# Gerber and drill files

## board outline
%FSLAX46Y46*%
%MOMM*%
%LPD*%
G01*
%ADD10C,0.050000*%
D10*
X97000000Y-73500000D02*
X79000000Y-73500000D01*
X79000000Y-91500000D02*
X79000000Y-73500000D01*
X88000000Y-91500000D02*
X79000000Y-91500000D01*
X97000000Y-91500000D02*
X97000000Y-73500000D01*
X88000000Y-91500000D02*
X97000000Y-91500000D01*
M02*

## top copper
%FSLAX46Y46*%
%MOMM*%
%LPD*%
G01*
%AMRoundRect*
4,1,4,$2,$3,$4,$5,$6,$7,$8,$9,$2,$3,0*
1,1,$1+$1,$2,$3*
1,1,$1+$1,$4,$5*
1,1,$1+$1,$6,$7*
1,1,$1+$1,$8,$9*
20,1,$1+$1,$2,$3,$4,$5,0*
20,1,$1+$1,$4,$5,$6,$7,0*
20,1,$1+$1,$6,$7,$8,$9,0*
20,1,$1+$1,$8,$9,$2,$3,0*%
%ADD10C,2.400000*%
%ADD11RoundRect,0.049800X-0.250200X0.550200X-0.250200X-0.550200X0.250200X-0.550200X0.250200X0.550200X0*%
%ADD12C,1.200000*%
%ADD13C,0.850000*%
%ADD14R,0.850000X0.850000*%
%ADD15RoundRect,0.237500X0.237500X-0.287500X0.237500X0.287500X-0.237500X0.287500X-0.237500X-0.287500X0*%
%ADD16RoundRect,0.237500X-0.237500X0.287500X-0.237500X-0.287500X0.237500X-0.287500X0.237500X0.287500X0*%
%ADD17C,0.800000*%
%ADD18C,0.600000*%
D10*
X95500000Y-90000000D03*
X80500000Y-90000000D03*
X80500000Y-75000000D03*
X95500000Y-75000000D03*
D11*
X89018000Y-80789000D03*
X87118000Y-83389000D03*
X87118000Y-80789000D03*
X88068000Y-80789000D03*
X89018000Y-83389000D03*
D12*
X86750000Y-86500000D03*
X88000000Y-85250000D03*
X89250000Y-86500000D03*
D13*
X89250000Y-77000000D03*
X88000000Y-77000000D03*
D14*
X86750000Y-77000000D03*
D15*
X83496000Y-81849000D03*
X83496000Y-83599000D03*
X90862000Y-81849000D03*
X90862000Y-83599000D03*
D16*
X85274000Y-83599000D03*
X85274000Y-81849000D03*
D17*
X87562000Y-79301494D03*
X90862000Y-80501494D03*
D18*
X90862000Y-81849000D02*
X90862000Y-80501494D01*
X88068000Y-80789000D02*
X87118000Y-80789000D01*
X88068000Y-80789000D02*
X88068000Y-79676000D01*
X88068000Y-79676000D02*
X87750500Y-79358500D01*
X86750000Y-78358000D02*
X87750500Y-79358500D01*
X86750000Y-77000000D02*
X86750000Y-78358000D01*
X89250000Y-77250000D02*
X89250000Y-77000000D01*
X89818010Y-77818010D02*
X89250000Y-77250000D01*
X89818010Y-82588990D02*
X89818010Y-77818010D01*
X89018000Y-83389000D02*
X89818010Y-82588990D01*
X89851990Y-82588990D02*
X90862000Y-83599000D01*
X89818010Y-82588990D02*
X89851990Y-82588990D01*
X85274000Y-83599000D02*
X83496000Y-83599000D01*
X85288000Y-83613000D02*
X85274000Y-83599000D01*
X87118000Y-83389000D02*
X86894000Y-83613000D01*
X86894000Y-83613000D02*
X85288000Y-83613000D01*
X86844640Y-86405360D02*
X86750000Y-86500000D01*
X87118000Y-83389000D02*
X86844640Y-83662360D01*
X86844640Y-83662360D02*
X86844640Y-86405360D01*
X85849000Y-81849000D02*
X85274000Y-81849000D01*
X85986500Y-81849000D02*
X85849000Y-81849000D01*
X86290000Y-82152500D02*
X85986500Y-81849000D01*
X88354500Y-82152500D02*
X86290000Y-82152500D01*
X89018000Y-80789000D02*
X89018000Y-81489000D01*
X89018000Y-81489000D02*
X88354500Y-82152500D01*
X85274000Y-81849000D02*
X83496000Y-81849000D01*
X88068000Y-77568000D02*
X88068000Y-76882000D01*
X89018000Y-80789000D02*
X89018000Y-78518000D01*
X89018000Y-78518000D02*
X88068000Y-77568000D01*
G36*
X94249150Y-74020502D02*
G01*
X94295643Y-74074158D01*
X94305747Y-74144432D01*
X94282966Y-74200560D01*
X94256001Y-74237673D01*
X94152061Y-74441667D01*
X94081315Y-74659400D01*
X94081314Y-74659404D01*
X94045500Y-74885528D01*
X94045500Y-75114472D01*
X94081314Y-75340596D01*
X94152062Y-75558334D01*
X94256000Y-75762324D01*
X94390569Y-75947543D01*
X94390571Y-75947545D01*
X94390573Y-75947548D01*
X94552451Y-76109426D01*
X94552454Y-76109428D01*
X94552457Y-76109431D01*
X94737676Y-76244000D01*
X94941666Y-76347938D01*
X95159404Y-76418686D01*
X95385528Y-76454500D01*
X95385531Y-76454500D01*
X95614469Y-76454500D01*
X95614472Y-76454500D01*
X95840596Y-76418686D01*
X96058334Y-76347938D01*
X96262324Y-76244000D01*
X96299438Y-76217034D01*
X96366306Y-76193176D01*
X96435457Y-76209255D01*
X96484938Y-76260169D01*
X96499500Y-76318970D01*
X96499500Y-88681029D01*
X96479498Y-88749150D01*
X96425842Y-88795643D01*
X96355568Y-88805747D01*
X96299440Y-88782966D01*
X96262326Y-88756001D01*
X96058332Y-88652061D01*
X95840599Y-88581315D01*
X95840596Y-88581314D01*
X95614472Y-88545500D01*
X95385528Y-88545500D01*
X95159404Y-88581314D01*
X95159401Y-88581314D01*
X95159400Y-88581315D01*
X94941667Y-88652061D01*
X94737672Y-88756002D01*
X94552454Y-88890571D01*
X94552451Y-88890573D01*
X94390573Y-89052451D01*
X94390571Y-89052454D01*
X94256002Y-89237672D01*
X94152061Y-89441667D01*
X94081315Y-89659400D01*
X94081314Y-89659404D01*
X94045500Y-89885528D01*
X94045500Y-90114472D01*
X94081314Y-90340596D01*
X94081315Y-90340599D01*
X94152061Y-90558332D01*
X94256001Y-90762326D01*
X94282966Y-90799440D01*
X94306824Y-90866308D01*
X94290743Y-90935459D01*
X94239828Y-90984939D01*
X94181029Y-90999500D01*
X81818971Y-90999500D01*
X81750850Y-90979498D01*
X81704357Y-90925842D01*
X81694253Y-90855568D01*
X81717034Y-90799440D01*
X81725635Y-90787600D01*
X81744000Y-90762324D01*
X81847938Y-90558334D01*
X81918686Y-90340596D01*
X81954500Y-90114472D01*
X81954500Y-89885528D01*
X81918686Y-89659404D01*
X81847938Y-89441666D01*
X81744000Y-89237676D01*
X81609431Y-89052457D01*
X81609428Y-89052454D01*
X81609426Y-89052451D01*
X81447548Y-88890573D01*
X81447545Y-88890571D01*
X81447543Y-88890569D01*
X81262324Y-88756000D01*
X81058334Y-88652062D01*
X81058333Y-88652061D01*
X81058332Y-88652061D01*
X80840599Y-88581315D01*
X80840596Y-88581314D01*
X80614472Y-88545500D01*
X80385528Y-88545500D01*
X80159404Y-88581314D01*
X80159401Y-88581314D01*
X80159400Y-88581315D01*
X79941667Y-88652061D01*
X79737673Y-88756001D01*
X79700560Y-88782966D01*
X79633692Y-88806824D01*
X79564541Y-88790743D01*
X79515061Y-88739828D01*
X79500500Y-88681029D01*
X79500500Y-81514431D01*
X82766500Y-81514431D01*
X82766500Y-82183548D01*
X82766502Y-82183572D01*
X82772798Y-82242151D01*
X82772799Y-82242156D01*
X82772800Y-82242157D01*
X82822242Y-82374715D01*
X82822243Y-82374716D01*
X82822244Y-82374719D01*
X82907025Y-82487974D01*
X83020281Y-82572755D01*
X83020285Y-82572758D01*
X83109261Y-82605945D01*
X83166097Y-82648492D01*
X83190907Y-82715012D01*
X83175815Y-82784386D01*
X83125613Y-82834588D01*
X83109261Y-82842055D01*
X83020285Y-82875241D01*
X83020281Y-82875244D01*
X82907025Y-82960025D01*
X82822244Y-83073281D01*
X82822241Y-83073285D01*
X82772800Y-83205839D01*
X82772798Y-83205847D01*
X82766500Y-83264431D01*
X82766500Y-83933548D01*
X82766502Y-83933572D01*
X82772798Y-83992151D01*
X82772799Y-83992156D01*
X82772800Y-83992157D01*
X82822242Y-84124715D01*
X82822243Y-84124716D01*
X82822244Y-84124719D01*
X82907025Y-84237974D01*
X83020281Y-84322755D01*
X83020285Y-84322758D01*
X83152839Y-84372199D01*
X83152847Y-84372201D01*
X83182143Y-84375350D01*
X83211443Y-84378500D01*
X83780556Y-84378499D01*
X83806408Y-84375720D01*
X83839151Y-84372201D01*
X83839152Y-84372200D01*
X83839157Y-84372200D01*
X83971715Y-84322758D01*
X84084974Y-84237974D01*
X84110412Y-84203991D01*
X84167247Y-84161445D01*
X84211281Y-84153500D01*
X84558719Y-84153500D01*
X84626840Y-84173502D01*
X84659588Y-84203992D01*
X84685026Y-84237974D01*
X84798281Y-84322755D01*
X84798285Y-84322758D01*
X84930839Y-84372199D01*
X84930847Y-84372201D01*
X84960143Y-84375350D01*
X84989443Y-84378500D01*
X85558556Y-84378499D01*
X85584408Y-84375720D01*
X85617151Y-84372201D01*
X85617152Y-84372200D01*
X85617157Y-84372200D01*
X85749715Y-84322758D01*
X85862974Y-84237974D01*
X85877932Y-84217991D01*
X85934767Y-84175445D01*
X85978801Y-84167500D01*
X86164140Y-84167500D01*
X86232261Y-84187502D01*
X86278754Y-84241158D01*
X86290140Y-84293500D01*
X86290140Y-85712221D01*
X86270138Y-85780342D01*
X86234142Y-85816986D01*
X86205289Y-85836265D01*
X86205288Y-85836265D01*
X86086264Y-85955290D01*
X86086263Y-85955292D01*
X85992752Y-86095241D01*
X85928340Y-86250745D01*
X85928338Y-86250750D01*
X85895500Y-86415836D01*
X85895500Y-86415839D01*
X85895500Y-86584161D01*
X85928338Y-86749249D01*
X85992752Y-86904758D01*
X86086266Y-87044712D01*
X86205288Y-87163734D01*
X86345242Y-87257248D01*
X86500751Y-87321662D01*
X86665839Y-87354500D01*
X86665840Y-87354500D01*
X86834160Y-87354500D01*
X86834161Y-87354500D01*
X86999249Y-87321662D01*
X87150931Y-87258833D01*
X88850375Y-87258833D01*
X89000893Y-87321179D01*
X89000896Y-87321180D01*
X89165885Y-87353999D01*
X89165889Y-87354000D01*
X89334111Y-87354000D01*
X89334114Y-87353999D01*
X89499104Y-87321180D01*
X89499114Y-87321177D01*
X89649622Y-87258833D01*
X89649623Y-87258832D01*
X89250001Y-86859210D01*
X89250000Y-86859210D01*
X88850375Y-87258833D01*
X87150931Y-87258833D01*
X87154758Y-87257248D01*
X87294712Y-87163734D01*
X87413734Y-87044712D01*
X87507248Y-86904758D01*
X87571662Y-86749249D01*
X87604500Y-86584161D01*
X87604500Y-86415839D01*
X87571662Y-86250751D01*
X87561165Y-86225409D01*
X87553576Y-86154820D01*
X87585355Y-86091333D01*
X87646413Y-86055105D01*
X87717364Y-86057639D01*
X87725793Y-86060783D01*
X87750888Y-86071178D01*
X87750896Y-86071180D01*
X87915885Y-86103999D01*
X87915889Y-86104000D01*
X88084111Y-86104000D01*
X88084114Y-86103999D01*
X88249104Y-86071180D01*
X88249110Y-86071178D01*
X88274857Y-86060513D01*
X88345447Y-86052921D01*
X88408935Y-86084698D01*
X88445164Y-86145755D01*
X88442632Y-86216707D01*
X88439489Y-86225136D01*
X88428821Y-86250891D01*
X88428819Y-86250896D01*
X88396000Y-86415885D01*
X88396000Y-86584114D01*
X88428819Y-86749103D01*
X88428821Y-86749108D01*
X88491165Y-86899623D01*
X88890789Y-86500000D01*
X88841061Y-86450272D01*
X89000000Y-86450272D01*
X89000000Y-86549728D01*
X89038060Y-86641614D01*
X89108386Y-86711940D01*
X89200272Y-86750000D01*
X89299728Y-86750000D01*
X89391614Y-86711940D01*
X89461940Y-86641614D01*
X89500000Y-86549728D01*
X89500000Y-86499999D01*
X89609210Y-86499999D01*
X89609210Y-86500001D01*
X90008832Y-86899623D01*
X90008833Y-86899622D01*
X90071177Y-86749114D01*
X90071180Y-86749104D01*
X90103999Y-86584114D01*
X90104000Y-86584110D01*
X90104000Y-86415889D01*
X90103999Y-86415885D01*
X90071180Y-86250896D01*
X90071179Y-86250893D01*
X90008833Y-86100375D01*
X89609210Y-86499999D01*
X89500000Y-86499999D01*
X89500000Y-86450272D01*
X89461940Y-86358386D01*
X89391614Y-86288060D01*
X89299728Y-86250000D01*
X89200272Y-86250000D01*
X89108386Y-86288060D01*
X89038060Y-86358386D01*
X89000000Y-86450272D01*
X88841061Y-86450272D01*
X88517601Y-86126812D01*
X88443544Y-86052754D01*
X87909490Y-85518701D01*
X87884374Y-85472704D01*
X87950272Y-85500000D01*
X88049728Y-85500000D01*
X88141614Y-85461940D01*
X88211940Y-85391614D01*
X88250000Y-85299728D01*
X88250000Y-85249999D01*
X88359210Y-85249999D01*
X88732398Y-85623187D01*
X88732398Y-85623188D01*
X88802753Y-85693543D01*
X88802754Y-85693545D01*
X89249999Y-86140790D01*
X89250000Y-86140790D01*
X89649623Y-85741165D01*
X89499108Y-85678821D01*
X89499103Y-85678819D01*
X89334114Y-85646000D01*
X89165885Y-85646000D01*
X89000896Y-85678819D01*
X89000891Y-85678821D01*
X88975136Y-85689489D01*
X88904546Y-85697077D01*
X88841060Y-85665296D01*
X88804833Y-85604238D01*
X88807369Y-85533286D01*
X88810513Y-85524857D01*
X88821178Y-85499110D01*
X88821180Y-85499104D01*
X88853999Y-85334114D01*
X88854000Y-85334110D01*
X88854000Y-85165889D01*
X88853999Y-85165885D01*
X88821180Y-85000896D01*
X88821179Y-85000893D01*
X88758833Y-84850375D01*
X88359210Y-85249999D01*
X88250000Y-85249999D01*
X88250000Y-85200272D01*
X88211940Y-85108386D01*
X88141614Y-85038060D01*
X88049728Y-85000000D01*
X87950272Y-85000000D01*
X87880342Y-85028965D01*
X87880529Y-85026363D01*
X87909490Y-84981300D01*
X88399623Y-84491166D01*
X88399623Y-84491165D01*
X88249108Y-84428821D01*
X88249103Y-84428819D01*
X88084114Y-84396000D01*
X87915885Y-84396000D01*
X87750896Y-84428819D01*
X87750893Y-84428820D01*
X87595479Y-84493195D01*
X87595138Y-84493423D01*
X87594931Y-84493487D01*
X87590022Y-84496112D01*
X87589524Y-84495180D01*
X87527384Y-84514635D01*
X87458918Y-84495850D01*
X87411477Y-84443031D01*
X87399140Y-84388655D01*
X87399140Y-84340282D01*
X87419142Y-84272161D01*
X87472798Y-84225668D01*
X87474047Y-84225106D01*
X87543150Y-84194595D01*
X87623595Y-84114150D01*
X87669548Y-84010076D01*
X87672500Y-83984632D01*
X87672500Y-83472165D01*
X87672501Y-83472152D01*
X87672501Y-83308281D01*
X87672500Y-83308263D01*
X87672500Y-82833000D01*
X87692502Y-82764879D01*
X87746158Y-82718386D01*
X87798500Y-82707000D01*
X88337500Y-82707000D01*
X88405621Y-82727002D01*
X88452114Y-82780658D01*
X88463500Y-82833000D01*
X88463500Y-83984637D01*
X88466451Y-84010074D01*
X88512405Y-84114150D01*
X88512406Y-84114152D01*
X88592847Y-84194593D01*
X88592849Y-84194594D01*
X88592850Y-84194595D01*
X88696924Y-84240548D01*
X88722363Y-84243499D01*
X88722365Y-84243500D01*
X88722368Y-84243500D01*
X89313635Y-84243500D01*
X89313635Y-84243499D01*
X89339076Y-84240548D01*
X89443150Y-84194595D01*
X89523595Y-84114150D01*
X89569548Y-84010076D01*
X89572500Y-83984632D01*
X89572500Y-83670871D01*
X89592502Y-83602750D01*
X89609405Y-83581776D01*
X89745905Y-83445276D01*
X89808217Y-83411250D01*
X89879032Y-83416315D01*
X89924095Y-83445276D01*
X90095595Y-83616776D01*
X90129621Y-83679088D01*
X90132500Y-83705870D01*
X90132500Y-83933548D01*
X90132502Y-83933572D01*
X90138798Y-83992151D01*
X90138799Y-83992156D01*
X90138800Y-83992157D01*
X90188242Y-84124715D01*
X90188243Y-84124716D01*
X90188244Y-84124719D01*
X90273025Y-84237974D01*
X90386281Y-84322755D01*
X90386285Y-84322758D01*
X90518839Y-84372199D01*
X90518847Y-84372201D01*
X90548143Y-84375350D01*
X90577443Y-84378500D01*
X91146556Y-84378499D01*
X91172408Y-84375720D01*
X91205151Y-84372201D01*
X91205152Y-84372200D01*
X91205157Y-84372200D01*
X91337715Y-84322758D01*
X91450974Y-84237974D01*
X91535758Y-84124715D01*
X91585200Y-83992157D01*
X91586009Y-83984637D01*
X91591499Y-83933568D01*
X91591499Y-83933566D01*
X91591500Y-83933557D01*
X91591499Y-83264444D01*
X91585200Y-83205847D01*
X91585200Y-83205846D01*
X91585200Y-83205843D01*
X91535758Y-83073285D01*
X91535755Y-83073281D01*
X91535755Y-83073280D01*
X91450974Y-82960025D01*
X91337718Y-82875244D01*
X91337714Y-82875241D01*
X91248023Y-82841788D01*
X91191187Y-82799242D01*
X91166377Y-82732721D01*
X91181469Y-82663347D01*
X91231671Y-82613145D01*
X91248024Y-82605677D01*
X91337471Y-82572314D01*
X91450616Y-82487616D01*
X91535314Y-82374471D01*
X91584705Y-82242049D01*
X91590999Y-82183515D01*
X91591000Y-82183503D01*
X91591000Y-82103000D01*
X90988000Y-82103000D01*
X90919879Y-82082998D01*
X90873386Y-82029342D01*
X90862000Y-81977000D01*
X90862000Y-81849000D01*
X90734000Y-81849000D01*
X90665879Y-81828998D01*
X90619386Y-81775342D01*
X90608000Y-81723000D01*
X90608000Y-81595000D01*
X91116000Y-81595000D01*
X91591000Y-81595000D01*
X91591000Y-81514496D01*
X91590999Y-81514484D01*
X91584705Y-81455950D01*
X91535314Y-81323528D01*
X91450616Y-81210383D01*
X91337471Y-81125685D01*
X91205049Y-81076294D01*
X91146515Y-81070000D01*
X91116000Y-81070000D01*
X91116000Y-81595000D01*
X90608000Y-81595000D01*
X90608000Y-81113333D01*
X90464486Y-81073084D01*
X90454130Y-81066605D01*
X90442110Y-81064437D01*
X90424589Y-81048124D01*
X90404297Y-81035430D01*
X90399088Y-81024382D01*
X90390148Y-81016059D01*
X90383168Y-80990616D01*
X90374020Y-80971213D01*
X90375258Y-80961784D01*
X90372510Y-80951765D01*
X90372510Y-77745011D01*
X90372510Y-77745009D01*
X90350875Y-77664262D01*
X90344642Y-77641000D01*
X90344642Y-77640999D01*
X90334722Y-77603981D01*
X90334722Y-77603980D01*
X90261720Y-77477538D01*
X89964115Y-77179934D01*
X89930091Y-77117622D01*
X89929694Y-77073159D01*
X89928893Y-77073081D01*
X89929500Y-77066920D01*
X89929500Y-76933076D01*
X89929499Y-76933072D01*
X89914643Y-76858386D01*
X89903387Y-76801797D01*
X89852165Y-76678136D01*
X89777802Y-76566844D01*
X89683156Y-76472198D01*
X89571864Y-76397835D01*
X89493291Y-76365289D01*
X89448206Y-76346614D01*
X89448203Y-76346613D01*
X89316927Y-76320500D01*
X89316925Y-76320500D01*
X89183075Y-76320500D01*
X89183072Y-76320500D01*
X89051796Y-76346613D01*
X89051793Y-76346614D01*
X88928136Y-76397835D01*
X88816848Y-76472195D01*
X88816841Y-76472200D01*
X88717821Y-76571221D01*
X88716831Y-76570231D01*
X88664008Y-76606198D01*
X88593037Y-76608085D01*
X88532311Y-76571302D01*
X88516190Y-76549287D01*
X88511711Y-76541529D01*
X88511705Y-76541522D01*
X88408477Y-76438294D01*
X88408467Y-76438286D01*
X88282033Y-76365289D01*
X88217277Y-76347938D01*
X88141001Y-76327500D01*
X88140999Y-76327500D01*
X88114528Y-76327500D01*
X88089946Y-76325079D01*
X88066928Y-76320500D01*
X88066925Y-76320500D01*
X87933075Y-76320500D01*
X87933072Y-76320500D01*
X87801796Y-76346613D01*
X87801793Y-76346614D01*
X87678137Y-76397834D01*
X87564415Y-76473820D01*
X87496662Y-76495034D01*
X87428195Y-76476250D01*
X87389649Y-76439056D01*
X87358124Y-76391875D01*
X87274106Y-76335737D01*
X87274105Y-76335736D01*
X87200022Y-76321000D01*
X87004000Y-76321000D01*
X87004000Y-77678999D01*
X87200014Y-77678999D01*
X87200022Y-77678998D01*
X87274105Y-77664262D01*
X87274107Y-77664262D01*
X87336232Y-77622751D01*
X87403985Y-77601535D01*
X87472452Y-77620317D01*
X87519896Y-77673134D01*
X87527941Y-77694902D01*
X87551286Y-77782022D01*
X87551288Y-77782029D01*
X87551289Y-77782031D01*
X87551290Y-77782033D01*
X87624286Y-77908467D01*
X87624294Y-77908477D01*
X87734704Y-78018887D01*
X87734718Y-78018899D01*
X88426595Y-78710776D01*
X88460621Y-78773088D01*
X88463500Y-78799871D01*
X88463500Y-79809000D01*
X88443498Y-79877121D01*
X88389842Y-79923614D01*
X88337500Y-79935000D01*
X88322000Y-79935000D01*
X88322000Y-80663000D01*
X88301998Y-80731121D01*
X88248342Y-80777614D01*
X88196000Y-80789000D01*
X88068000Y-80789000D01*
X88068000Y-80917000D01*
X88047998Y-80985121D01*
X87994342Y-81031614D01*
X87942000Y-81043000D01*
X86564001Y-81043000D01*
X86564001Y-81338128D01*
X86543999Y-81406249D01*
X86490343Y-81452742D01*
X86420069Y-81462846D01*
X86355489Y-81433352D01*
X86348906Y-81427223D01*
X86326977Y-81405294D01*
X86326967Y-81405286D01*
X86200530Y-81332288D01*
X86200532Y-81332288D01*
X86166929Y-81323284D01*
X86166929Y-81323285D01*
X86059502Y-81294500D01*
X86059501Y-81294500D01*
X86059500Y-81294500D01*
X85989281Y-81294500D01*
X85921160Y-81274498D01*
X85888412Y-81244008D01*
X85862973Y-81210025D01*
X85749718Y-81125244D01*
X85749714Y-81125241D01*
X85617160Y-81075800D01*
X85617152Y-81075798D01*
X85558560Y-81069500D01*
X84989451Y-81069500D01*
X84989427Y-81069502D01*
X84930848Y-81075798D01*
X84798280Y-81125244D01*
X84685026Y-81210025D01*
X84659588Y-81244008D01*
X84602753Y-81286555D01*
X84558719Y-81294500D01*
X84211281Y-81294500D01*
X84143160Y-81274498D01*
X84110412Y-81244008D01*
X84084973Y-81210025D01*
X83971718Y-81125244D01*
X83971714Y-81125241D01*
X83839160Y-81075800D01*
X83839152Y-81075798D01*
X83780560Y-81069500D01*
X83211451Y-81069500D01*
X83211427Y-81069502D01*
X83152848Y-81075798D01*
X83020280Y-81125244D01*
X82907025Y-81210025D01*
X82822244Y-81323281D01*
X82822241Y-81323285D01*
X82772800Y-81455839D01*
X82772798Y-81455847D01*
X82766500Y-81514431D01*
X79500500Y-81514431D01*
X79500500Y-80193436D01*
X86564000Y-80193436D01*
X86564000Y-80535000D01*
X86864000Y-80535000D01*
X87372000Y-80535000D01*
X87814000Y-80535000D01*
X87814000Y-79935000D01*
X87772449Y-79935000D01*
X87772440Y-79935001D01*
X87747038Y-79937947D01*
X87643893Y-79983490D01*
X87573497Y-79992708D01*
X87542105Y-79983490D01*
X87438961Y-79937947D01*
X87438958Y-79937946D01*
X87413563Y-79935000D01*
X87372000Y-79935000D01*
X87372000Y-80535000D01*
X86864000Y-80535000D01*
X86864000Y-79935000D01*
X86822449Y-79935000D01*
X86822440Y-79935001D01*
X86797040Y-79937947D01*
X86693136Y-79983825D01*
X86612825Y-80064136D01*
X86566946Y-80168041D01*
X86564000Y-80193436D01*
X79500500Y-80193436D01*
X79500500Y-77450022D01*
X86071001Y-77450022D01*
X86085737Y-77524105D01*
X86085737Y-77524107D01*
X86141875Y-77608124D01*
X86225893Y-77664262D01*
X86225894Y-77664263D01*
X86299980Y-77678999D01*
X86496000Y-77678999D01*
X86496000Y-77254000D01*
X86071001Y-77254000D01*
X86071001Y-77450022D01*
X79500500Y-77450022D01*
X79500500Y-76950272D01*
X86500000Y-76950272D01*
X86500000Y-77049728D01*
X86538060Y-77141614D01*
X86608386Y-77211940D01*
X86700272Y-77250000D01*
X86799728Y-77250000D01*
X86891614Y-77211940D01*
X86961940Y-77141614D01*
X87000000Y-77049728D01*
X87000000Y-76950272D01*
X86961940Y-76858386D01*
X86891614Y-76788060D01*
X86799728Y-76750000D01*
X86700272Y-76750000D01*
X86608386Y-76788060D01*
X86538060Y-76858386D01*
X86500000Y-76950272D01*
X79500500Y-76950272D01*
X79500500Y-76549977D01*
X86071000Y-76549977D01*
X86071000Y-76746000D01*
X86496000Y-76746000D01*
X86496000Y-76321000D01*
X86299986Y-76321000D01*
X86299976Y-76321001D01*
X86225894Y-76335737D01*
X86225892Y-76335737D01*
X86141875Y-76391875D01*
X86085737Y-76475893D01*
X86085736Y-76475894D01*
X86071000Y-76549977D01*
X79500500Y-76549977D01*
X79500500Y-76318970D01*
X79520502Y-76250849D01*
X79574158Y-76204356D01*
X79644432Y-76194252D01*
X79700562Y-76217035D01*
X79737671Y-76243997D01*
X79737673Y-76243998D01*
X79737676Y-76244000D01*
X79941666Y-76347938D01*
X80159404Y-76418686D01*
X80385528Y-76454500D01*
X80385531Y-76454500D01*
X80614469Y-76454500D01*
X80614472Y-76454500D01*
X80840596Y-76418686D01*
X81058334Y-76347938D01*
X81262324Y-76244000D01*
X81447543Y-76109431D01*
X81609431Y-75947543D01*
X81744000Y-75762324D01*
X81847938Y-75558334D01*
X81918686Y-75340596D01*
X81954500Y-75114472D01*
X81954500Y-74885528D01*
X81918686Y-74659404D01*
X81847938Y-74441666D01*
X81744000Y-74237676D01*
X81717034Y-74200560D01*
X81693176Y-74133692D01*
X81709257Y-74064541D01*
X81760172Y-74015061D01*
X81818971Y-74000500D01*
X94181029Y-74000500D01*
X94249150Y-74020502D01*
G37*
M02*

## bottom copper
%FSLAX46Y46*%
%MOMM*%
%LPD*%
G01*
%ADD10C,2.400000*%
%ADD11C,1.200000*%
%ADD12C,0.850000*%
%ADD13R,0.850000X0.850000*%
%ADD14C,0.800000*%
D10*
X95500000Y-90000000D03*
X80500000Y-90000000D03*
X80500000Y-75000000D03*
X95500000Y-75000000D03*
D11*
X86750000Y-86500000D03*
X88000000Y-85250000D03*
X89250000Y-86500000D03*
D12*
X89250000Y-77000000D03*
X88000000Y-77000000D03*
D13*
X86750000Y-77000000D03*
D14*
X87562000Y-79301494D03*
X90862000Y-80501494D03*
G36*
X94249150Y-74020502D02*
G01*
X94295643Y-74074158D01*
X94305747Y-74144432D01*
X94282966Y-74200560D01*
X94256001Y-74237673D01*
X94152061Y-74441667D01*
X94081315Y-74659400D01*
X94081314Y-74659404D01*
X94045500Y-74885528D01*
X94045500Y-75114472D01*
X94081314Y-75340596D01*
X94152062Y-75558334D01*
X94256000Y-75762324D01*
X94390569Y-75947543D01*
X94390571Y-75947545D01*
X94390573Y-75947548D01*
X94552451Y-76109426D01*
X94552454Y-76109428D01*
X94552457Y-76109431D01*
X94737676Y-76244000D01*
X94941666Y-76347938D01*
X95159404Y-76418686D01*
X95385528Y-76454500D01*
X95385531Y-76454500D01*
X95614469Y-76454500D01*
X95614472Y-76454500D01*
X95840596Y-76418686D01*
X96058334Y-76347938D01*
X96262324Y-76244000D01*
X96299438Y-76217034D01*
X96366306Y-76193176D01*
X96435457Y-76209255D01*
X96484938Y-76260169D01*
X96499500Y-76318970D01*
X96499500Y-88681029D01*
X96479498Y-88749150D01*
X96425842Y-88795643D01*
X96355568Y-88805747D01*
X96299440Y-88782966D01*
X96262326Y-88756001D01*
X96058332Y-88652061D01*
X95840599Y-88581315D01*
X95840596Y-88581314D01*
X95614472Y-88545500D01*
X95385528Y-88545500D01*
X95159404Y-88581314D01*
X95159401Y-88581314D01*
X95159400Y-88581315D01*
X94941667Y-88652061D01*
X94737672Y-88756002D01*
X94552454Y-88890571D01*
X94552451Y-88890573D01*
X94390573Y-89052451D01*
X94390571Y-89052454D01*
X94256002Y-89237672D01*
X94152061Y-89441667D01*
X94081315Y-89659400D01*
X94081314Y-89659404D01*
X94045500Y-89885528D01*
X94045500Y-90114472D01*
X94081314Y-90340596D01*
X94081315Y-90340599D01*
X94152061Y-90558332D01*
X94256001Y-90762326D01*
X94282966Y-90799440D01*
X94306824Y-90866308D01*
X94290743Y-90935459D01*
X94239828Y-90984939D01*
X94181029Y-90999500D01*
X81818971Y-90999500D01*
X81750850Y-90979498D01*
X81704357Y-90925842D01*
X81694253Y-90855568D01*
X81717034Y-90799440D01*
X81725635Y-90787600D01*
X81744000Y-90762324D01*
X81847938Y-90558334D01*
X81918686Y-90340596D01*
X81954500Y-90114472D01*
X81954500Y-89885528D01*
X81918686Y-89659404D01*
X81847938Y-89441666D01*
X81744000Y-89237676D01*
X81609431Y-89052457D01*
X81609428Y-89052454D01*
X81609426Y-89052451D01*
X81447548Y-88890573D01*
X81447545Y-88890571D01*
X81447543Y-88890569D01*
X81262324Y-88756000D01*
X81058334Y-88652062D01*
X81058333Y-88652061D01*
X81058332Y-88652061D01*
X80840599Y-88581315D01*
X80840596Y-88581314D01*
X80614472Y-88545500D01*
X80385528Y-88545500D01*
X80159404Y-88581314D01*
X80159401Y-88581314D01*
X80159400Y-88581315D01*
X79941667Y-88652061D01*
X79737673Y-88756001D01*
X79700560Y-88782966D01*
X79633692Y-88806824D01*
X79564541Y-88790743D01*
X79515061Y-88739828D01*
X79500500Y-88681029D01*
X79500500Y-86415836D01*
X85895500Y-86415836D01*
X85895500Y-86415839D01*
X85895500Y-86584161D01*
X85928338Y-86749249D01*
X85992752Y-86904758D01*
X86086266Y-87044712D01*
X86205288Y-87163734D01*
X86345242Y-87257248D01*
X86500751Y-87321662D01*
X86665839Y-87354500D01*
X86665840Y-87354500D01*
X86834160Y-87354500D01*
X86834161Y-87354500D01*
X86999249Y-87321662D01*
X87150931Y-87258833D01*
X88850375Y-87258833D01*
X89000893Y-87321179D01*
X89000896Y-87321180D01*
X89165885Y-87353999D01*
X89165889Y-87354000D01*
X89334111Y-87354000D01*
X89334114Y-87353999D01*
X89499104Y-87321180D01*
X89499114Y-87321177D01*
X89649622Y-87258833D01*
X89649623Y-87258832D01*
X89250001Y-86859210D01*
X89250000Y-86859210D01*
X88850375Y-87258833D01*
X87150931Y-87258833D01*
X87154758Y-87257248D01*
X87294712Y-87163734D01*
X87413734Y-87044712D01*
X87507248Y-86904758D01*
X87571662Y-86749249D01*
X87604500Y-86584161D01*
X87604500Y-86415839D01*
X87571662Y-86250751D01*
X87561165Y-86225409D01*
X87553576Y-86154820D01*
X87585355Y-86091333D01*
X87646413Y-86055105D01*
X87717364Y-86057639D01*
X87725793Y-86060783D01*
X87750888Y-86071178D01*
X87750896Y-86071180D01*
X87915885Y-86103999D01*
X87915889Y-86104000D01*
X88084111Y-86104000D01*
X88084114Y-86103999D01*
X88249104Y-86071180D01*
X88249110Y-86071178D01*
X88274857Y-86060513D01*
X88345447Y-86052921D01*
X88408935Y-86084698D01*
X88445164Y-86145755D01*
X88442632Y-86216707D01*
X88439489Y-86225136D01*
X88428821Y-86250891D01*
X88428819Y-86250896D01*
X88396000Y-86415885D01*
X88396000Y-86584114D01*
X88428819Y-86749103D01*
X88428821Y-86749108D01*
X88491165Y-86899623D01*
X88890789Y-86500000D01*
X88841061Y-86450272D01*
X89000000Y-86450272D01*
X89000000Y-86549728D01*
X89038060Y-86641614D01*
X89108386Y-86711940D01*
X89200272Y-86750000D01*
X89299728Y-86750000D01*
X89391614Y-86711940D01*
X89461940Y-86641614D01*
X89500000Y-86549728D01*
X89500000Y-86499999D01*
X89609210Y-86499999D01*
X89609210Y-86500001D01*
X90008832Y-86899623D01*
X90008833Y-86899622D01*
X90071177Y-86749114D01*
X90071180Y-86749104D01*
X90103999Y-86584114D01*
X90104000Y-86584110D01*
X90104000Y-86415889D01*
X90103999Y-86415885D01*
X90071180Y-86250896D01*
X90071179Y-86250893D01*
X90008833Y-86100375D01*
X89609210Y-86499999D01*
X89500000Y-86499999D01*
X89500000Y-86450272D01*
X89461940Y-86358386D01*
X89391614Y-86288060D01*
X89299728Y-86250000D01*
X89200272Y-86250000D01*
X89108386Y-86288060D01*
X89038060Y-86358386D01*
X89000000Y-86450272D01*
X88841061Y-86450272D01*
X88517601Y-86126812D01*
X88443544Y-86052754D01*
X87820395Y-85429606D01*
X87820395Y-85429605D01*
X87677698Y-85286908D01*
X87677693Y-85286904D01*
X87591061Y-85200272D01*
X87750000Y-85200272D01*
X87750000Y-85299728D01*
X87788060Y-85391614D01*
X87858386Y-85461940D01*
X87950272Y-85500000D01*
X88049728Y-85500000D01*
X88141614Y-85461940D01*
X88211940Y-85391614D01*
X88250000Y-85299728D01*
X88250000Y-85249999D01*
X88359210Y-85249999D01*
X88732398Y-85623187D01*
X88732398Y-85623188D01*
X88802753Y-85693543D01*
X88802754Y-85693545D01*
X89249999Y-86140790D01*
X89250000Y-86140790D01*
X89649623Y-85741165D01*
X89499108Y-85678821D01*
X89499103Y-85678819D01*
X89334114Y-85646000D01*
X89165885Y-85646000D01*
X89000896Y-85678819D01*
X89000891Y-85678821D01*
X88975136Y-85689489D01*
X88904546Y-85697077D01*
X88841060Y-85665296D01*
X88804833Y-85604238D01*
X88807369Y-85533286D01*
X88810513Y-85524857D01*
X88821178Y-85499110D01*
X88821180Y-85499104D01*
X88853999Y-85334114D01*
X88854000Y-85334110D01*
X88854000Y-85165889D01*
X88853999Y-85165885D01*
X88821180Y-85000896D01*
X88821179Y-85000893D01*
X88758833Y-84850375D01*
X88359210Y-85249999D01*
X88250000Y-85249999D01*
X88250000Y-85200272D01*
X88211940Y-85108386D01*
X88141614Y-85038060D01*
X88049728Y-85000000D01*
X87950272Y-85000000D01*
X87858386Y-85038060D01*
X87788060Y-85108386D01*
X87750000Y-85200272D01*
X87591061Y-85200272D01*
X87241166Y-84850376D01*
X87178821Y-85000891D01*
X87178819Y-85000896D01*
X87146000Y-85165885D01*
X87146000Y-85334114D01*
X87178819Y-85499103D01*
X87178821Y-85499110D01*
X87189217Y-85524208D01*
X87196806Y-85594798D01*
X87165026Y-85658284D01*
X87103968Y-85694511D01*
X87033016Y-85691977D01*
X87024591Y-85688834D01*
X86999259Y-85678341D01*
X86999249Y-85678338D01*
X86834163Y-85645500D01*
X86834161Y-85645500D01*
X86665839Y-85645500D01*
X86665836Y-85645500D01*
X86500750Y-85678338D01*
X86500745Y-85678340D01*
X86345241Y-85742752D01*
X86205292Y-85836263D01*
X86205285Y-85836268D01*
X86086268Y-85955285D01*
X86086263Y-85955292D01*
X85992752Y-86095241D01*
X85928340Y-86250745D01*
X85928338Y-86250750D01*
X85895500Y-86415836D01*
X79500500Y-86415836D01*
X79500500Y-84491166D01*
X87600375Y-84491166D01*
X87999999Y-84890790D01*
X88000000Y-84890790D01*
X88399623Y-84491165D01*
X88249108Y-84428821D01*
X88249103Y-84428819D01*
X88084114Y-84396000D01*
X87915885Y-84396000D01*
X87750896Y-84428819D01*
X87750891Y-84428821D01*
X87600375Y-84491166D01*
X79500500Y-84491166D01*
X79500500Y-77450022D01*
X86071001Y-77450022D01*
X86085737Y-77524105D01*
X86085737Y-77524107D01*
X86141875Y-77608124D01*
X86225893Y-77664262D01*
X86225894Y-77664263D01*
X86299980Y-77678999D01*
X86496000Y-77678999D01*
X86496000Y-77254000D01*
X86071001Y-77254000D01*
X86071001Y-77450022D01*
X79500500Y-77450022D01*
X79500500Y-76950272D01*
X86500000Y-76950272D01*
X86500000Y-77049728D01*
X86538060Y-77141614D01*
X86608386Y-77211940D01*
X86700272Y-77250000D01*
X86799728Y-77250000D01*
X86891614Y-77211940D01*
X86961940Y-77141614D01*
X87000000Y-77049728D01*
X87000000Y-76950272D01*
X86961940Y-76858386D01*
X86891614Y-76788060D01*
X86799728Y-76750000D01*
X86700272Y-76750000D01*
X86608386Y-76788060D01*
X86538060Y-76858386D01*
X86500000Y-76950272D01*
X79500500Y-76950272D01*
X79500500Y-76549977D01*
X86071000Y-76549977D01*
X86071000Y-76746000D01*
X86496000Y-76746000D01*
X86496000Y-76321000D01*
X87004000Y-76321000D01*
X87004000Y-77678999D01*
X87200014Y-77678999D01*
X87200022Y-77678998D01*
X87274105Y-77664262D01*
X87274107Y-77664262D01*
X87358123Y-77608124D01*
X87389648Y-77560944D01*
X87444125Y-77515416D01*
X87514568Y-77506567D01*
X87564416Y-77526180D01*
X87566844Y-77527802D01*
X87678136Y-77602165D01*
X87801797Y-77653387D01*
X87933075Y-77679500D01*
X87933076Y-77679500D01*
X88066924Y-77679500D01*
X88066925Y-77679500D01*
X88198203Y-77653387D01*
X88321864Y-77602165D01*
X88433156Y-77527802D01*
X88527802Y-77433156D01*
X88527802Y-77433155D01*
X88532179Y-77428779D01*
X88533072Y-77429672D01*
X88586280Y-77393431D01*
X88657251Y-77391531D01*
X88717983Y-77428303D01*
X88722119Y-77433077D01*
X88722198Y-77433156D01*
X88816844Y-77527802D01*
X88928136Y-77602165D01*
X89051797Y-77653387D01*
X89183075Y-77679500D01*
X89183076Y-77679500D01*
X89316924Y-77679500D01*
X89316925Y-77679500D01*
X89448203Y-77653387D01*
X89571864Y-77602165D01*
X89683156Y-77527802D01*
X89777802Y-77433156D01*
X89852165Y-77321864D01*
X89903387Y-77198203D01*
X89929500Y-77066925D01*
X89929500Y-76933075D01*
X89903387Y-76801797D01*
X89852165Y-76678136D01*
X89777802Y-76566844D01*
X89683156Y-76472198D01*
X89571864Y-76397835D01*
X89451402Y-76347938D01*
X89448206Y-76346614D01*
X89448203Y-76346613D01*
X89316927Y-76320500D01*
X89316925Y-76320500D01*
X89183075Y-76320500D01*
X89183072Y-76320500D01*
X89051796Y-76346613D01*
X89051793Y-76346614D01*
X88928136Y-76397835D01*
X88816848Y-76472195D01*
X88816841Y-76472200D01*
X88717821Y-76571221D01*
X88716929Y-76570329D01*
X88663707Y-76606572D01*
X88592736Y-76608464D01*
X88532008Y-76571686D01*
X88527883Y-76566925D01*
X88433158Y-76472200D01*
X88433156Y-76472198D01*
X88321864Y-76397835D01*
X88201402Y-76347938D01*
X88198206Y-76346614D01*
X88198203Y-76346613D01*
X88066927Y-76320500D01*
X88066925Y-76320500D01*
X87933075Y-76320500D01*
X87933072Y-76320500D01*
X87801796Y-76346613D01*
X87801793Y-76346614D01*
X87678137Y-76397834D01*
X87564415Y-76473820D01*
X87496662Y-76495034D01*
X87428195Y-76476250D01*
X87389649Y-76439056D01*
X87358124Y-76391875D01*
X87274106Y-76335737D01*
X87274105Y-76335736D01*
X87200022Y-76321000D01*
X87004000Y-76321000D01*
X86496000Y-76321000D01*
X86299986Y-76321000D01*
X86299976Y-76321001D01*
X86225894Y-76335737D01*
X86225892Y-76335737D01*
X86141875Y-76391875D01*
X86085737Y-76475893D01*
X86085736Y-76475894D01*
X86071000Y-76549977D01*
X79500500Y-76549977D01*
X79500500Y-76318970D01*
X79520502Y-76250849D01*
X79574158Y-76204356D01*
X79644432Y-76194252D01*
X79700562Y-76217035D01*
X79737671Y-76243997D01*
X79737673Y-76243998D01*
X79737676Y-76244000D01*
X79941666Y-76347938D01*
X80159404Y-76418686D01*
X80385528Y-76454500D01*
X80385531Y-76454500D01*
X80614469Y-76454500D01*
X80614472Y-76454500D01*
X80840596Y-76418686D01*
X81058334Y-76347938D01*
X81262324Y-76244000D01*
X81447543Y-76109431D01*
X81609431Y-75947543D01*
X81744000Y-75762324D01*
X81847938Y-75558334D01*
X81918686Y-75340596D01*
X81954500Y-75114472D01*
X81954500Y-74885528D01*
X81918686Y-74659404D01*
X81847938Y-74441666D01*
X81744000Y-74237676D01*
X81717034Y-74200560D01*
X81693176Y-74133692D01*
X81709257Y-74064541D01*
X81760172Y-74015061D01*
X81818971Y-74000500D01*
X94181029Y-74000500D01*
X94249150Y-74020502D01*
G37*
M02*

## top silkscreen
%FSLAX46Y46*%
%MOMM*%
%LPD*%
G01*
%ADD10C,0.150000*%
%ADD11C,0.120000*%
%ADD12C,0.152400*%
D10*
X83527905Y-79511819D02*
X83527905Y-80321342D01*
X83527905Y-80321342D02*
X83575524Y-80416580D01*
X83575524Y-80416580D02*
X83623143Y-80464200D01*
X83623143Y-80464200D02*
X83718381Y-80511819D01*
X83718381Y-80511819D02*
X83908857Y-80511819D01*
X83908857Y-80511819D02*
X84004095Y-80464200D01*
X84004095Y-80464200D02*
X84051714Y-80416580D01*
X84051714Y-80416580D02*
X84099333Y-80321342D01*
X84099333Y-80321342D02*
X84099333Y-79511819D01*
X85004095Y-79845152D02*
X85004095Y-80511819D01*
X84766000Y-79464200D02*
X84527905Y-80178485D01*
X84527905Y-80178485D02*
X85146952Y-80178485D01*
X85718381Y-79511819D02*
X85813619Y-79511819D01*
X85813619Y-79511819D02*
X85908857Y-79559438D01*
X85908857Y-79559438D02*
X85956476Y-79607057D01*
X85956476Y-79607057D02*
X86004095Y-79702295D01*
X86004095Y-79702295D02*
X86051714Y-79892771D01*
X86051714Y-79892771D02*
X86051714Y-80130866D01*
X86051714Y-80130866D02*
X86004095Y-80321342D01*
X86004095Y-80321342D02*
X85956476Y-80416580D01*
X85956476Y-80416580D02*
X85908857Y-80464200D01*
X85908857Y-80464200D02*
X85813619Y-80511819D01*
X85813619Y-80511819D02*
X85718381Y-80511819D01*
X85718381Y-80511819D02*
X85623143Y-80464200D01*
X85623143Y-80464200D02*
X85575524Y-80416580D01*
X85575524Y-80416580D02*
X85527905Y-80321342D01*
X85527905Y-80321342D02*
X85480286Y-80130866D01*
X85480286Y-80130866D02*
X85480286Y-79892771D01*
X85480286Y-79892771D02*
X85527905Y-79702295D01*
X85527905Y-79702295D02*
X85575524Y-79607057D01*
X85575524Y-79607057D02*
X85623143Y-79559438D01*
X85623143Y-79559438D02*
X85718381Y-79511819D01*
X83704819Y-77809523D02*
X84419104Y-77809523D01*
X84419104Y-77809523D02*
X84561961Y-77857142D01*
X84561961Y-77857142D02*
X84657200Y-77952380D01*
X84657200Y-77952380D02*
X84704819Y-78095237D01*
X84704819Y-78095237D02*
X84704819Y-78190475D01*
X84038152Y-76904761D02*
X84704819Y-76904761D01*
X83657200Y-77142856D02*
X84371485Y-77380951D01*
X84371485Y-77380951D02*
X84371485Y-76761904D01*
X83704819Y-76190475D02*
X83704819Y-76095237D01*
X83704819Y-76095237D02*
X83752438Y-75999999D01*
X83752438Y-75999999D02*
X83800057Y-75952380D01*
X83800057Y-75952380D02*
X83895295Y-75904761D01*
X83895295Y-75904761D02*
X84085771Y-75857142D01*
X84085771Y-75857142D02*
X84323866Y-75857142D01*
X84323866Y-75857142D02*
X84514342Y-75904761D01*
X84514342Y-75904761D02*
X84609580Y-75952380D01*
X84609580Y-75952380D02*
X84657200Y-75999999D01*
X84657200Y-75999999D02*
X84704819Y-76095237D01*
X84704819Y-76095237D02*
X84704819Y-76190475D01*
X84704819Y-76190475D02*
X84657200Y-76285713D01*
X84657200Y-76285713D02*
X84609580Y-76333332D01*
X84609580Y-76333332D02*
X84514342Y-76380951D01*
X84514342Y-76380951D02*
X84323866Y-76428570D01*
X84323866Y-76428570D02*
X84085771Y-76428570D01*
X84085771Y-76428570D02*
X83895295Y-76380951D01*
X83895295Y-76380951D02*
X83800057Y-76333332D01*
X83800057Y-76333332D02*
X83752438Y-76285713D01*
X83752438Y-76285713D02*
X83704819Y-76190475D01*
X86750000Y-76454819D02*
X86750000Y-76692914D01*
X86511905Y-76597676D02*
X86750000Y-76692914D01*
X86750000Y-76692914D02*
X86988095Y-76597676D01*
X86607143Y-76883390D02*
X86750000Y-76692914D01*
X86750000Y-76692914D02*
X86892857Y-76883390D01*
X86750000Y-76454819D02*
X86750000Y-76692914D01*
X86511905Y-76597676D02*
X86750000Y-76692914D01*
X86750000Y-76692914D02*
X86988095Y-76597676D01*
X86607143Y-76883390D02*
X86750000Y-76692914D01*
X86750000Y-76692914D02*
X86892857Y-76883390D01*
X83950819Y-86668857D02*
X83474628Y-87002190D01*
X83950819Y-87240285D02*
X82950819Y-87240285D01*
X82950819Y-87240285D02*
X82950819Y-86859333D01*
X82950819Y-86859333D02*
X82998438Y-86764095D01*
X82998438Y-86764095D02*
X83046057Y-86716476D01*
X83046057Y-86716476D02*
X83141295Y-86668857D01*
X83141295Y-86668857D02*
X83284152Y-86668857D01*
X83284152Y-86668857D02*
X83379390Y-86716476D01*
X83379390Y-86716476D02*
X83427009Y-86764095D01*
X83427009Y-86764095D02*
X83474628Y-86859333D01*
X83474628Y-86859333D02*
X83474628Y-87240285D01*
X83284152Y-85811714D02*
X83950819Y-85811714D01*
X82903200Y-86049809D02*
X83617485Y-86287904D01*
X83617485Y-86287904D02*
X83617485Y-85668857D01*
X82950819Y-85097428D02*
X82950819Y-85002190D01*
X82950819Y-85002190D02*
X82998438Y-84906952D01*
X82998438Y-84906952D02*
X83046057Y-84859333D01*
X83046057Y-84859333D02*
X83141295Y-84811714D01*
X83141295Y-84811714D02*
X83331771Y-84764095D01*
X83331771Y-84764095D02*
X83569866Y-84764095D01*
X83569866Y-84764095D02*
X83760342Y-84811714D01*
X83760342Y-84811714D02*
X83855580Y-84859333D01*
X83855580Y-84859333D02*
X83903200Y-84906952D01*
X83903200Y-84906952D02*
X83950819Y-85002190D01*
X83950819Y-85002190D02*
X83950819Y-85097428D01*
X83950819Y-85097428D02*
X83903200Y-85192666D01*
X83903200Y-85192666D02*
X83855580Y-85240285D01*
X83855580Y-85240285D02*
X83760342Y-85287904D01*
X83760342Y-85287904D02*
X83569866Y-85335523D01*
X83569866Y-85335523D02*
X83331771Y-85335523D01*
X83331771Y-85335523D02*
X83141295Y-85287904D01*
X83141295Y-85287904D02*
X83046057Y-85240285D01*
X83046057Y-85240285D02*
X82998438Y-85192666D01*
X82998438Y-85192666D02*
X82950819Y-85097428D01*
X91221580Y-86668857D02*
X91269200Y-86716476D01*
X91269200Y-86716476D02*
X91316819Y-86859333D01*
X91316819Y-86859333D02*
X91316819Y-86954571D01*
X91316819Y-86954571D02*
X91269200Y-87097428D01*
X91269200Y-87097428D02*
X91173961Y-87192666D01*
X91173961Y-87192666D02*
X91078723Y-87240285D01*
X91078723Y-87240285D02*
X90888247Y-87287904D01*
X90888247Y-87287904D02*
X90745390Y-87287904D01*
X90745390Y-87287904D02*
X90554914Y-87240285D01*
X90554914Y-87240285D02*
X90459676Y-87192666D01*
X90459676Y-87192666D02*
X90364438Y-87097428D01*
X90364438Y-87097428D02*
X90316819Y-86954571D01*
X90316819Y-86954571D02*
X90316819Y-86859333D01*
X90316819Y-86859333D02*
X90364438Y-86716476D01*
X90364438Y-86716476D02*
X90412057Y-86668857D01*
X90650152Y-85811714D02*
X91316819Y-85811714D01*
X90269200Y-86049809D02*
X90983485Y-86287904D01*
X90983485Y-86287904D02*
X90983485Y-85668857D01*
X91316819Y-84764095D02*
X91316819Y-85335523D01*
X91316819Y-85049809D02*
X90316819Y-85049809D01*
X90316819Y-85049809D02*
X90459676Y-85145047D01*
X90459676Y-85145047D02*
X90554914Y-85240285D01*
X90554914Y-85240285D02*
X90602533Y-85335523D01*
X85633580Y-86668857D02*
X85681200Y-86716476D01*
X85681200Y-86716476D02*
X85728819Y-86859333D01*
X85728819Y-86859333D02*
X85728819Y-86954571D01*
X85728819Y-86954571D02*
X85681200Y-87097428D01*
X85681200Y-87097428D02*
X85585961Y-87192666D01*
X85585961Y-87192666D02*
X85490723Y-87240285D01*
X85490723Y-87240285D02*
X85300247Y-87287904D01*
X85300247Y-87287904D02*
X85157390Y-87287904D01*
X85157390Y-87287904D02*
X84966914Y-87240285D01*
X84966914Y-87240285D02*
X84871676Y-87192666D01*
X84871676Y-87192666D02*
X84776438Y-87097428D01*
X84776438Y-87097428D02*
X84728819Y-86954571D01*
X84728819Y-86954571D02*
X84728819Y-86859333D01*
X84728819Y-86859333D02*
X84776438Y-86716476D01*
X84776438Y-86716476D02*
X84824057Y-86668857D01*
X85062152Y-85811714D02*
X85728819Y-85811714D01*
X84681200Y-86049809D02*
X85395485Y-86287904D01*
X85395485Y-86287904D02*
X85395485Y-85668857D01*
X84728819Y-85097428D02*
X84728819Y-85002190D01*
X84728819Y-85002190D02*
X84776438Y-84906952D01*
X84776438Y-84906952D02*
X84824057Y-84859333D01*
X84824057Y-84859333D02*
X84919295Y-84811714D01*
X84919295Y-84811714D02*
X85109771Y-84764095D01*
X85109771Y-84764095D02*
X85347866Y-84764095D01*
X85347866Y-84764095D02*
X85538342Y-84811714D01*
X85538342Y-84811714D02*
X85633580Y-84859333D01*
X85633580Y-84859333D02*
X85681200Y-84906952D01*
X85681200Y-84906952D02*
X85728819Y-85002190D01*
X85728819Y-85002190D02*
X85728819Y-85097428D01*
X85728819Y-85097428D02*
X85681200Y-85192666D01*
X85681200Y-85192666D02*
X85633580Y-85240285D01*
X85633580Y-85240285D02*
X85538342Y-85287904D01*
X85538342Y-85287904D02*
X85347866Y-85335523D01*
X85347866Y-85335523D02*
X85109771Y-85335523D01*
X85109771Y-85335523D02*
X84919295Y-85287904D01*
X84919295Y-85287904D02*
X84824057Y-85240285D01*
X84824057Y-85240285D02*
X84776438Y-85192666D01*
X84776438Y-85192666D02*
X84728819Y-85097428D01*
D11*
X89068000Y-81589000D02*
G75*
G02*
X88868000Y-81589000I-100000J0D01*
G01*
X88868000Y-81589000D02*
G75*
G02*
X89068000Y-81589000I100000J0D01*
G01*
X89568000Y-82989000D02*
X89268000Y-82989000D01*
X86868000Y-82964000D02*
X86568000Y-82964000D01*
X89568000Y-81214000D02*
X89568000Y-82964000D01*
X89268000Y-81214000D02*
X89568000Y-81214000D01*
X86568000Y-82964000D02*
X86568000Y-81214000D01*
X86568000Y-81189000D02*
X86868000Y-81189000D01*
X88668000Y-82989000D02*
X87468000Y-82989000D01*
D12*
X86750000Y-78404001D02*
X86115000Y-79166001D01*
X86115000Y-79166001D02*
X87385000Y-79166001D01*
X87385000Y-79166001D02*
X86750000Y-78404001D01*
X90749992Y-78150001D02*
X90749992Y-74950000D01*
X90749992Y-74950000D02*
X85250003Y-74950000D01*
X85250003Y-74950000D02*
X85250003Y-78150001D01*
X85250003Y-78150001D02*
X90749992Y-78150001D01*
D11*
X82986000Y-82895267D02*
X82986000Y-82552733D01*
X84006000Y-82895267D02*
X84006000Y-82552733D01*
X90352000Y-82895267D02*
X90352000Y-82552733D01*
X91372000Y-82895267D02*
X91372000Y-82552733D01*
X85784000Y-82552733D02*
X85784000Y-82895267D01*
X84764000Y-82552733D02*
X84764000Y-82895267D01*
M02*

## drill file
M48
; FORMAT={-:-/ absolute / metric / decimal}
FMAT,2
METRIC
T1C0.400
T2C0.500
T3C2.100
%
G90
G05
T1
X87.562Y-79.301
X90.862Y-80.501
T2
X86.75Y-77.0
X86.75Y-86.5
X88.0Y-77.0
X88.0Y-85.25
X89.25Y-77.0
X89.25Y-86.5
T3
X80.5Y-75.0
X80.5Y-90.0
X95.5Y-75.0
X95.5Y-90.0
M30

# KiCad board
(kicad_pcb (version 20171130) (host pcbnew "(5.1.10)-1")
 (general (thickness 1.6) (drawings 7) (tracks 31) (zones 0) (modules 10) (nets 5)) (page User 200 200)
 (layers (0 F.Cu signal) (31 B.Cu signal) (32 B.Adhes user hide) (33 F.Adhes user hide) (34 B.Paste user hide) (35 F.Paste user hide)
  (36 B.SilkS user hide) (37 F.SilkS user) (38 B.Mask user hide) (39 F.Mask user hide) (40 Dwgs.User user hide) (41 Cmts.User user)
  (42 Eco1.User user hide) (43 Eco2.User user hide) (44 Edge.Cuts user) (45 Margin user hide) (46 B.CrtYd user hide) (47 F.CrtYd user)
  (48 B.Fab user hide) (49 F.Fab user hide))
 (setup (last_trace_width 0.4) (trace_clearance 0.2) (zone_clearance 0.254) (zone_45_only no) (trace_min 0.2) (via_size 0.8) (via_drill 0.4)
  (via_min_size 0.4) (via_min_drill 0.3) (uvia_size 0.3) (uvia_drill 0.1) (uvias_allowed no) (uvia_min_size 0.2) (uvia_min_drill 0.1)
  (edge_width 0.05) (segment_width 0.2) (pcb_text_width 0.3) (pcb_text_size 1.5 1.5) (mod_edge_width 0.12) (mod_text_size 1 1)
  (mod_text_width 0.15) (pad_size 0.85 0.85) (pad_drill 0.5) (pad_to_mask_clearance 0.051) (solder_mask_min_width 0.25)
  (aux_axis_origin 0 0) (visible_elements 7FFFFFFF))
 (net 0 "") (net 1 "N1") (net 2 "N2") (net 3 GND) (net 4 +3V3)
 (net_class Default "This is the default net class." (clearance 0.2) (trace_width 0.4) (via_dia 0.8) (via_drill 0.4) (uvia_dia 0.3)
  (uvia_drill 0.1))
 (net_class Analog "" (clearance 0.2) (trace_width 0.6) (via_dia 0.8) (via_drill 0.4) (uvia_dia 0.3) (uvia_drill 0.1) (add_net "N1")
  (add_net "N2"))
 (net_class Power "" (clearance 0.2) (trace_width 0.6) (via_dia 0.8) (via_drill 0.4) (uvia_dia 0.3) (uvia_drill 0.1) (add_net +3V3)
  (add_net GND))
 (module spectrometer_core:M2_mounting (layer F.Cu) (at 95.5 90)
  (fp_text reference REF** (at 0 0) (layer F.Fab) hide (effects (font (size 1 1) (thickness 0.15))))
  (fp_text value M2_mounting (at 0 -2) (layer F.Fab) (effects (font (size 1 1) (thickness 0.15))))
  (pad "" np_thru_hole circle (at 0 0) (size 2.4 2.4) (drill 2.1) (layers *.Cu *.Mask) (zone_connect 0)))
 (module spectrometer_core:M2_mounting (layer F.Cu) (at 80.5 90)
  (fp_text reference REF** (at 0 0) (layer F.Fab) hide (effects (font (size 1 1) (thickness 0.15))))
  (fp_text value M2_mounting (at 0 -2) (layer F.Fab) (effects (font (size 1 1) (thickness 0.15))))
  (pad "" np_thru_hole circle (at 0 0) (size 2.4 2.4) (drill 2.1) (layers *.Cu *.Mask) (zone_connect 0)))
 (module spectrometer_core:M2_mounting (layer F.Cu) (at 80.5 75)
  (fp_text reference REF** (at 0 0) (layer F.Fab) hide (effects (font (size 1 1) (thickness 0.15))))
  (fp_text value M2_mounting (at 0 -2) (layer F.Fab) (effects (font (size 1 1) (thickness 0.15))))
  (pad "" np_thru_hole circle (at 0 0) (size 2.4 2.4) (drill 2.1) (layers *.Cu *.Mask) (zone_connect 0)))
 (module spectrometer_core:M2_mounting (layer F.Cu) (at 95.5 75)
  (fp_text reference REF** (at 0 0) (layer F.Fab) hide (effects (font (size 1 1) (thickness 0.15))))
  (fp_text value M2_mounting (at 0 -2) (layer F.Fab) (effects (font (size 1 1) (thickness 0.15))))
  (pad "" np_thru_hole circle (at 0 0) (size 2.4 2.4) (drill 2.1) (layers *.Cu *.Mask) (zone_connect 0)))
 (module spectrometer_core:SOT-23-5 (layer F.Cu) (at 88.068 82.089 270)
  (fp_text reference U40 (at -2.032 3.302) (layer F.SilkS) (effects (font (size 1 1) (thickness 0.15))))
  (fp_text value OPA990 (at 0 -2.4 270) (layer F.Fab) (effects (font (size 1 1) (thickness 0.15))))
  (fp_circle (center -0.5 -0.9) (end -0.4 -0.9) (layer F.SilkS) (width 0.12))
  (fp_line (start 0.9 -1.5) (end 0.9 -1.2) (layer F.SilkS) (width 0.12))
  (fp_line (start 0.875 1.2) (end 0.875 1.5) (layer F.SilkS) (width 0.12))
  (fp_line (start -0.875 -1.5) (end 0.875 -1.5) (layer F.SilkS) (width 0.12))
  (fp_line (start -0.875 -1.2) (end -0.875 -1.5) (layer F.SilkS) (width 0.12))
  (fp_line (start 0.875 1.5) (end -0.875 1.5) (layer F.SilkS) (width 0.12))
  (fp_line (start -0.9 1.5) (end -0.9 1.2) (layer F.SilkS) (width 0.12))
  (fp_line (start 0.9 -0.6) (end 0.9 0.6) (layer F.SilkS) (width 0.12))
  (pad 1 smd roundrect (at -1.3 -0.95 270) (size 1.2 0.6) (layers F.Cu F.Paste F.Mask) (roundrect_rratio 0.083) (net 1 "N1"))
  (pad 4 smd roundrect (at 1.3 0.95 270) (size 1.2 0.6) (layers F.Cu F.Paste F.Mask) (roundrect_rratio 0.083) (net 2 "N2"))
  (pad 3 smd roundrect (at -1.3 0.95 270) (size 1.2 0.6) (layers F.Cu F.Paste F.Mask) (roundrect_rratio 0.083) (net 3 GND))
  (pad 2 smd roundrect (at -1.3 0 270) (size 1.2 0.6) (layers F.Cu F.Paste F.Mask) (roundrect_rratio 0.083) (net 3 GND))
  (pad 5 smd roundrect (at 1.3 -0.95 270) (size 1.2 0.6) (layers F.Cu F.Paste F.Mask) (roundrect_rratio 0.083) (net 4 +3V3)))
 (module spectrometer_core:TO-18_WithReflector (layer B.Cu) (at 88 86.5 180)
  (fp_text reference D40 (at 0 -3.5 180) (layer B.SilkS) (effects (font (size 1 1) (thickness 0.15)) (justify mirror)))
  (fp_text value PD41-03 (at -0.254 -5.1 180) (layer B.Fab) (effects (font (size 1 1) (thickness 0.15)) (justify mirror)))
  (pad 2 thru_hole circle (at 1.25 0 180) (size 1.2 1.2) (drill 0.5) (layers *.Cu *.Mask) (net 2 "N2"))
  (pad 3 thru_hole circle (at 0 1.25 180) (size 1.2 1.2) (drill 0.5) (layers *.Cu *.Mask) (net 3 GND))
  (pad 1 thru_hole circle (at -1.25 0 180) (size 1.2 1.2) (drill 0.5) (layers *.Cu *.Mask) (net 3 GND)))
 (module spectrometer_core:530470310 (layer F.Cu) (at 86.75 77 180)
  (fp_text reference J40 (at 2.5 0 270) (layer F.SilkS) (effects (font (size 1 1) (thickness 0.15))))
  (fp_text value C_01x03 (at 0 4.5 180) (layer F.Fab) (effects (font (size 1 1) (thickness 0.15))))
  (fp_line (start 0 -1.404001) (end 0.635 -2.166001) (layer F.SilkS) (width 0.1524))
  (fp_line (start 0.635 -2.166001) (end -0.635 -2.166001) (layer F.SilkS) (width 0.1524))
  (fp_line (start -0.635 -2.166001) (end 0 -1.404001) (layer F.SilkS) (width 0.1524))
  (fp_line (start -3.999992 -1.150001) (end -3.999992 2.05) (layer F.SilkS) (width 0.1524))
  (fp_line (start -3.999992 2.05) (end 1.499997 2.05) (layer F.SilkS) (width 0.1524))
  (fp_line (start 1.499997 2.05) (end 1.499997 -1.150001) (layer F.SilkS) (width 0.1524))
  (fp_line (start 1.499997 -1.150001) (end -3.999992 -1.150001) (layer F.SilkS) (width 0.1524))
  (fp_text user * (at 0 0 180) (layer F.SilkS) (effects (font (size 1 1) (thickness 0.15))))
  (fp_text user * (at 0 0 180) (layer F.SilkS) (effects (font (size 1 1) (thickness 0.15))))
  (pad 3 thru_hole circle (at -2.5 0 180) (size 0.85 0.85) (drill 0.5) (layers *.Cu *.Mask) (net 4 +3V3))
  (pad 2 thru_hole circle (at -1.25 0 180) (size 0.85 0.85) (drill 0.5) (layers *.Cu *.Mask) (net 1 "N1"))
  (pad 1 thru_hole rect (at 0 0 180) (size 0.85 0.85) (drill 0.5) (layers *.Cu *.Mask) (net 3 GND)))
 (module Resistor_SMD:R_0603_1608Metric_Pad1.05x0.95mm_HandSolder (layer F.Cu) (at 83.496 82.724 90)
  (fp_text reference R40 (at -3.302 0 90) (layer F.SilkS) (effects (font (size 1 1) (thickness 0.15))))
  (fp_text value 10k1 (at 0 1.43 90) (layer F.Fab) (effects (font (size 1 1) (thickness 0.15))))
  (fp_line (start -0.171267 -0.51) (end 0.171267 -0.51) (layer F.SilkS) (width 0.12))
  (fp_line (start -0.171267 0.51) (end 0.171267 0.51) (layer F.SilkS) (width 0.12))
  (pad 2 smd roundrect (at 0.875 0 90) (size 1.05 0.95) (layers F.Cu F.Paste F.Mask) (roundrect_rratio 0.25) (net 1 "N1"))
  (pad 1 smd roundrect (at -0.875 0 90) (size 1.05 0.95) (layers F.Cu F.Paste F.Mask) (roundrect_rratio 0.25) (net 2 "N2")))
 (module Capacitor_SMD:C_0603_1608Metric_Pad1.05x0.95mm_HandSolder (layer F.Cu) (at 90.862 82.724 90)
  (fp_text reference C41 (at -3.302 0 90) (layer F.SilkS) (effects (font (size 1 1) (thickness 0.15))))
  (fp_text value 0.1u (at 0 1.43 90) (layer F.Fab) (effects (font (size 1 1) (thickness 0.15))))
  (fp_line (start -0.171267 -0.51) (end 0.171267 -0.51) (layer F.SilkS) (width 0.12))
  (fp_line (start -0.171267 0.51) (end 0.171267 0.51) (layer F.SilkS) (width 0.12))
  (pad 2 smd roundrect (at 0.875 0 90) (size 1.05 0.95) (layers F.Cu F.Paste F.Mask) (roundrect_rratio 0.25) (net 3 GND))
  (pad 1 smd roundrect (at -0.875 0 90) (size 1.05 0.95) (layers F.Cu F.Paste F.Mask) (roundrect_rratio 0.25) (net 4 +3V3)))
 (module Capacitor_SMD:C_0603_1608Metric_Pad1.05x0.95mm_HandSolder (layer F.Cu) (at 85.274 82.724 270)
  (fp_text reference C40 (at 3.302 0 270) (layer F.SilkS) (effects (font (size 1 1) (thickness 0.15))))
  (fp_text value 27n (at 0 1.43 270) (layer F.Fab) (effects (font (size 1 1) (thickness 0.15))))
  (fp_line (start -0.171267 -0.51) (end 0.171267 -0.51) (layer F.SilkS) (width 0.12))
  (fp_line (start -0.171267 0.51) (end 0.171267 0.51) (layer F.SilkS) (width 0.12))
  (pad 2 smd roundrect (at 0.875 0 270) (size 1.05 0.95) (layers F.Cu F.Paste F.Mask) (roundrect_rratio 0.25) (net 2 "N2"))
  (pad 1 smd roundrect (at -0.875 0 270) (size 1.05 0.95) (layers F.Cu F.Paste F.Mask) (roundrect_rratio 0.25) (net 1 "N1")))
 (gr_line (start 97 73.5) (end 79 73.5) (layer Edge.Cuts) (width 0.05))
 (gr_line (start 79 91.5) (end 79 73.5) (layer Edge.Cuts) (width 0.05))
 (gr_line (start 88 91.5) (end 79 91.5) (layer Edge.Cuts) (width 0.05))
 (gr_line (start 97 91.5) (end 97 73.5) (layer Edge.Cuts) (width 0.05))
 (gr_line (start 88 91.5) (end 97 91.5) (layer Edge.Cuts) (width 0.05))
 (via (at 87.562 79.301494) (size 0.8) (drill 0.4) (layers F.Cu B.Cu) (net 3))
 (via (at 90.862 80.501494) (size 0.8) (drill 0.4) (layers F.Cu B.Cu) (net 3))
 (segment (start 90.862 81.849) (end 90.862 80.501494) (width 0.6) (layer F.Cu) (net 3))
 (segment (start 88.068 80.789) (end 87.118 80.789) (width 0.6) (layer F.Cu) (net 3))
 (segment (start 88.068 80.789) (end 88.068 79.676) (width 0.6) (layer F.Cu) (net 3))
 (segment (start 88.068 79.676) (end 87.7505 79.3585) (width 0.6) (layer F.Cu) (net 3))
 (segment (start 86.75 78.358) (end 87.7505 79.3585) (width 0.6) (layer F.Cu) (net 3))
 (segment (start 86.75 77) (end 86.75 78.358) (width 0.6) (layer F.Cu) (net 3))
 (segment (start 89.25 77.25) (end 89.25 77) (width 0.6) (layer F.Cu) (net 4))
 (segment (start 89.81801 77.81801) (end 89.25 77.25) (width 0.6) (layer F.Cu) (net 4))
 (segment (start 89.81801 82.58899) (end 89.81801 77.81801) (width 0.6) (layer F.Cu) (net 4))
 (segment (start 89.018 83.389) (end 89.81801 82.58899) (width 0.6) (layer F.Cu) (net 4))
 (segment (start 89.85199 82.58899) (end 90.862 83.599) (width 0.6) (layer F.Cu) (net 4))
 (segment (start 89.81801 82.58899) (end 89.85199 82.58899) (width 0.6) (layer F.Cu) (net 4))
 (segment (start 85.274 83.599) (end 83.496 83.599) (width 0.6) (layer F.Cu) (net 2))
 (segment (start 85.288 83.613) (end 85.274 83.599) (width 0.6) (layer F.Cu) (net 2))
 (segment (start 87.118 83.389) (end 86.894 83.613) (width 0.6) (layer F.Cu) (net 2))
 (segment (start 86.894 83.613) (end 85.288 83.613) (width 0.6) (layer F.Cu) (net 2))
 (segment (start 86.84464 86.40536) (end 86.75 86.5) (width 0.6) (layer F.Cu) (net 2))
 (segment (start 87.118 83.389) (end 86.84464 83.66236) (width 0.6) (layer F.Cu) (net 2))
 (segment (start 86.84464 83.66236) (end 86.84464 86.40536) (width 0.6) (layer F.Cu) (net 2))
 (segment (start 85.849 81.849) (end 85.274 81.849) (width 0.6) (layer F.Cu) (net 1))
 (segment (start 85.9865 81.849) (end 85.849 81.849) (width 0.6) (layer F.Cu) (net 1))
 (segment (start 86.29 82.1525) (end 85.9865 81.849) (width 0.6) (layer F.Cu) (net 1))
 (segment (start 88.3545 82.1525) (end 86.29 82.1525) (width 0.6) (layer F.Cu) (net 1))
 (segment (start 89.018 80.789) (end 89.018 81.489) (width 0.6) (layer F.Cu) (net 1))
 (segment (start 89.018 81.489) (end 88.3545 82.1525) (width 0.6) (layer F.Cu) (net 1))
 (segment (start 85.274 81.849) (end 83.496 81.849) (width 0.6) (layer F.Cu) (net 1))
 (segment (start 88.068 77.568) (end 88.068 76.882) (width 0.6) (layer F.Cu) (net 1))
 (segment (start 89.018 80.789) (end 89.018 78.518) (width 0.6) (layer F.Cu) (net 1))
 (segment (start 89.018 78.518) (end 88.068 77.568) (width 0.6) (layer F.Cu) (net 1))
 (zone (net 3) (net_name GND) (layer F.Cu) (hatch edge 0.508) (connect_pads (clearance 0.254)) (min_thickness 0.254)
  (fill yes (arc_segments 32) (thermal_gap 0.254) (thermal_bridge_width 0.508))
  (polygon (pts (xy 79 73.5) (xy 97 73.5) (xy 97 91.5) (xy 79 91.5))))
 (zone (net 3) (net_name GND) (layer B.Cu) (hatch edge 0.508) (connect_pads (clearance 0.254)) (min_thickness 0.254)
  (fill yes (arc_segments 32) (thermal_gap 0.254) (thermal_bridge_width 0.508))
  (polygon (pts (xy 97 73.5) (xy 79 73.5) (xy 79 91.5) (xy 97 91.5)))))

